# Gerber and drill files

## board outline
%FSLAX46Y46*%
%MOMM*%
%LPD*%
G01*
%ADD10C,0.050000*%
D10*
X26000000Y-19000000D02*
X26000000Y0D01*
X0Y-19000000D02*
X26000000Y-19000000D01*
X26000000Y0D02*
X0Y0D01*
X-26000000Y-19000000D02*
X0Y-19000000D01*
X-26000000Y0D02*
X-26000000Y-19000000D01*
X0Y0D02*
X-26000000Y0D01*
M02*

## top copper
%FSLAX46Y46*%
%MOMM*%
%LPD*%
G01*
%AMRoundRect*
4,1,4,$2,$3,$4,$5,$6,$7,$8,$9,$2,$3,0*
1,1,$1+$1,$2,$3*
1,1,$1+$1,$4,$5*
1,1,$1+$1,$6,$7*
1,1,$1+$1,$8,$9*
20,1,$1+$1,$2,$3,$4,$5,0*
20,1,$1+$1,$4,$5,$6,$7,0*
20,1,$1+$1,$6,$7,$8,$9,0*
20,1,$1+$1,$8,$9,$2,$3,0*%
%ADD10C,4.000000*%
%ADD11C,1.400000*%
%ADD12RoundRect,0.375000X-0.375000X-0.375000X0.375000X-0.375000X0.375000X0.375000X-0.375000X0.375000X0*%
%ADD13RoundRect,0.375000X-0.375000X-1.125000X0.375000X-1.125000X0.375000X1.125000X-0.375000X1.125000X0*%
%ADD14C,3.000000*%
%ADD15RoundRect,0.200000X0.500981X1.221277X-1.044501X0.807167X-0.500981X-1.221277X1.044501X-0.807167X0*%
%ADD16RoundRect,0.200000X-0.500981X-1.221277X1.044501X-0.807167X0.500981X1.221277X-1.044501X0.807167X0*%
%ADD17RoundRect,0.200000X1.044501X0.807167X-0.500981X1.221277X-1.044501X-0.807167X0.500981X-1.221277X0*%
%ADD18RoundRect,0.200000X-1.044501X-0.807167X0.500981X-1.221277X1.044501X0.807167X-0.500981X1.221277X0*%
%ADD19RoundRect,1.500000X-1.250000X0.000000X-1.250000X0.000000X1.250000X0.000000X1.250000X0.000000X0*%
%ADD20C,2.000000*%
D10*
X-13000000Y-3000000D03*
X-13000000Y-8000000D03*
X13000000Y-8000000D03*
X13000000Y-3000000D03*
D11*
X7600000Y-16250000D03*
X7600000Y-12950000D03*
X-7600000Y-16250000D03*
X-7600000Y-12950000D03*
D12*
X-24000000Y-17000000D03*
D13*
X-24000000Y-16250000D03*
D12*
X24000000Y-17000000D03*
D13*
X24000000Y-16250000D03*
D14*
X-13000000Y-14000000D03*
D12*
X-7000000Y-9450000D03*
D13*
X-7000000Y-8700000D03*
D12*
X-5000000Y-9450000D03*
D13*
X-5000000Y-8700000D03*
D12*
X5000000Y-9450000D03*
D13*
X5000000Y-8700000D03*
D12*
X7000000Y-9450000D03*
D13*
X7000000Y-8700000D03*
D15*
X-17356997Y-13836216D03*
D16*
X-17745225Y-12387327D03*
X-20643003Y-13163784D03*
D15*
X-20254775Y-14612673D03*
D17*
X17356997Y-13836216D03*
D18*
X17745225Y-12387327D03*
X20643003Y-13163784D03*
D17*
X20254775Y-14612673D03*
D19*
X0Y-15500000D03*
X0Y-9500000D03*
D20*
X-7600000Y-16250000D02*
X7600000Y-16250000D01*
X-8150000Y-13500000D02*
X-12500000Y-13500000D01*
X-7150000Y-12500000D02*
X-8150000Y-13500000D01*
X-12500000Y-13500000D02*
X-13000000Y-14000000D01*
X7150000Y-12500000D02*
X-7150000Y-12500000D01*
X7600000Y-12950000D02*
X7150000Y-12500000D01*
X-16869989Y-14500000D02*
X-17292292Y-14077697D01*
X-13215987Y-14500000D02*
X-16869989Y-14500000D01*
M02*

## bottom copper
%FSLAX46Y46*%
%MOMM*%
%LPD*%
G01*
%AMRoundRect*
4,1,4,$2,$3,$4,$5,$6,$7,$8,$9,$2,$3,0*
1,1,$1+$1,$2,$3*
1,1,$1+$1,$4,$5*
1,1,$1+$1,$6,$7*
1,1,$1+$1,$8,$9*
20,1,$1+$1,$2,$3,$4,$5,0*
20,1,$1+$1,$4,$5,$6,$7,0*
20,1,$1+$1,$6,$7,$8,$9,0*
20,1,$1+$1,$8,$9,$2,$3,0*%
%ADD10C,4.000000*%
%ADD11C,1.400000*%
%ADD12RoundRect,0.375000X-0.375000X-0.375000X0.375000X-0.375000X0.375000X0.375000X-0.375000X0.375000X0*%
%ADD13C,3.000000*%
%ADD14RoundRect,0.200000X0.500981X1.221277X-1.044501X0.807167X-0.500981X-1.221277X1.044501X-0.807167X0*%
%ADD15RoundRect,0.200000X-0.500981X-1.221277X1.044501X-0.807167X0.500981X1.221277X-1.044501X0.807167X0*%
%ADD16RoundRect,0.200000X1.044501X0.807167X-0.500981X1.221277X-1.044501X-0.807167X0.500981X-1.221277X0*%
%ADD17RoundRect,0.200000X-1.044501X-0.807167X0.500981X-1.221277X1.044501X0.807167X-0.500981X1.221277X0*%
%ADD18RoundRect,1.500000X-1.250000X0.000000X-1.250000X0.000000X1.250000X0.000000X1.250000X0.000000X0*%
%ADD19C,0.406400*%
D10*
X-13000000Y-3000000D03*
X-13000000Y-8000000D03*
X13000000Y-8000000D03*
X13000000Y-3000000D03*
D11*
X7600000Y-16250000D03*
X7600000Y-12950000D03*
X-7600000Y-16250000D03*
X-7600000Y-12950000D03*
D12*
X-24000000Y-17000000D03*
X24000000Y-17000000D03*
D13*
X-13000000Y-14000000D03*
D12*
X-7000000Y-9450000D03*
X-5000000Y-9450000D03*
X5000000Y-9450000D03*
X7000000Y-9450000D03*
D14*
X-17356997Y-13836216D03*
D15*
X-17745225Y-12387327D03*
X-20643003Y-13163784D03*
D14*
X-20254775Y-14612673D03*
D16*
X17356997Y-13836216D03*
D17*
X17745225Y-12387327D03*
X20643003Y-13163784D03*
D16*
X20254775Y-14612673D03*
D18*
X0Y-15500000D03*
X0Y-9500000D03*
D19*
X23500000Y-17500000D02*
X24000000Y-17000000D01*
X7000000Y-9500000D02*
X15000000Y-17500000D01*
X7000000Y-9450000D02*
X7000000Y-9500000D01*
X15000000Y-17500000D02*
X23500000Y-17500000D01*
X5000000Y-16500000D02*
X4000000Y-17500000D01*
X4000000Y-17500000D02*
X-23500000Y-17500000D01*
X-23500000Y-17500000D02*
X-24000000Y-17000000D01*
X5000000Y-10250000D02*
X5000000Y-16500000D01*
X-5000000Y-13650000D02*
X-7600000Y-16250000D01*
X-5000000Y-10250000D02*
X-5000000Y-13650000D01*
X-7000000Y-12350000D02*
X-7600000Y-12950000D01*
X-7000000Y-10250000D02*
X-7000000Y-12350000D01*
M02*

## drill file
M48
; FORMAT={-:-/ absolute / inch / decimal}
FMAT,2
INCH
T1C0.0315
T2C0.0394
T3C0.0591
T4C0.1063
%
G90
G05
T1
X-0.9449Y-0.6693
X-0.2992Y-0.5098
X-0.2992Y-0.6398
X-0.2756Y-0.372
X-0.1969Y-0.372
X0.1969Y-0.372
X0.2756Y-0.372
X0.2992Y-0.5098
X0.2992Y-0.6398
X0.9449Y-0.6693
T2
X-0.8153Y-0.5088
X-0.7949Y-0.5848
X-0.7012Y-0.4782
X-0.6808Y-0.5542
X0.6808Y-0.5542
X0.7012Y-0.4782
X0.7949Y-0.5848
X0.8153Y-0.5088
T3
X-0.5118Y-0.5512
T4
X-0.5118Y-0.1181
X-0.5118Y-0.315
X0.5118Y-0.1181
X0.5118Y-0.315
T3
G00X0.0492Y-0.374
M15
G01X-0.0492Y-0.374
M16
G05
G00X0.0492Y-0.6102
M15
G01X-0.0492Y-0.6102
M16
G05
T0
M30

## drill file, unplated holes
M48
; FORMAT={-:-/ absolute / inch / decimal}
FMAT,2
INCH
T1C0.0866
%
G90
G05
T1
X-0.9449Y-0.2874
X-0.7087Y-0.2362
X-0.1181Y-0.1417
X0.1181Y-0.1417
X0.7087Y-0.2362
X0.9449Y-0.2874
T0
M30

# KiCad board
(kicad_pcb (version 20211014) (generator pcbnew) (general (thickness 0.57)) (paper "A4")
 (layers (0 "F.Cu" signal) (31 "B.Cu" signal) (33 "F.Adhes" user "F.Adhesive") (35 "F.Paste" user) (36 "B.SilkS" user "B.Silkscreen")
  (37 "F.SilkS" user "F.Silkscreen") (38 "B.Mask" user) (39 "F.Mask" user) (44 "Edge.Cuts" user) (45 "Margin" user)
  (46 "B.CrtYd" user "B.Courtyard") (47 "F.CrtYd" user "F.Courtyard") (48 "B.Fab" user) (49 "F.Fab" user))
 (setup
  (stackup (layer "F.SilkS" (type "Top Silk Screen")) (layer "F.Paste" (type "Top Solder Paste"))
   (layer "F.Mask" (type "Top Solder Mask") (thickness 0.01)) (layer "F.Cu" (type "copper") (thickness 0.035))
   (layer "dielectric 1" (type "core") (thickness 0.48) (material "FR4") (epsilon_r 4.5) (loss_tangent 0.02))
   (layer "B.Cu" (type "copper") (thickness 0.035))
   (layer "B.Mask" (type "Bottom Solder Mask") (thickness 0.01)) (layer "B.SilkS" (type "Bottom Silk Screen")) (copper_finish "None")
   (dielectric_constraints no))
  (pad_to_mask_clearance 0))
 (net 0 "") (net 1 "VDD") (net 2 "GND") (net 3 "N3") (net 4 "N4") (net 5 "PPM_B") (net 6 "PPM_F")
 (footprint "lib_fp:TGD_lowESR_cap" (layer "F.Cu") (at -7.6 14.6 90)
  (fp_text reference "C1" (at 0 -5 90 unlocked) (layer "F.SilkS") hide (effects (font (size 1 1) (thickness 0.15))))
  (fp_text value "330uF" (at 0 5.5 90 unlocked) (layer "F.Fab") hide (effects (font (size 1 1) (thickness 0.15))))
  (pad "1" thru_hole circle (at -1.65 0 90) (size 1.4 1.4) (drill 0.8) (layers *.Cu *.Mask) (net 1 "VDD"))
  (pad "2" thru_hole circle (at 1.65 0 90) (size 1.4 1.4) (drill 0.8) (layers *.Cu *.Mask) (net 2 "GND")))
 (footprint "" (layer "F.Cu") (at -13 14)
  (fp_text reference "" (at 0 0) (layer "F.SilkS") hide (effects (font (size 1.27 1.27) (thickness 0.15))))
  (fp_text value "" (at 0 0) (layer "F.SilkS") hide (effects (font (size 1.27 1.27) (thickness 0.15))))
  (pad "2" thru_hole circle (at 0 0 270) (size 3 3) (drill 1.5) (layers *.Cu *.Mask) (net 2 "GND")))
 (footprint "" (layer "F.Cu") (at 24 7.3)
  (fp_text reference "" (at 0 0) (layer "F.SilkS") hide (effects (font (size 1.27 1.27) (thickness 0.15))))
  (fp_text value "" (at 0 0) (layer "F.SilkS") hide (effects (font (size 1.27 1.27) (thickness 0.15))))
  (pad "" np_thru_hole circle (at 0 0 270) (size 2.2 2.2) (drill 2.2) (layers F&B.Cu *.Mask)))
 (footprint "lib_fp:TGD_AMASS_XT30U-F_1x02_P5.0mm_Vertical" (layer "F.Cu") (at 13 5.5 90)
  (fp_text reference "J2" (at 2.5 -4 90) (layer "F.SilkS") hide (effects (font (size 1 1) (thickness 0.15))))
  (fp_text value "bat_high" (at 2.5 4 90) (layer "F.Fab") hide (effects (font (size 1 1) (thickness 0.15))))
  (pad "1" thru_hole circle (at -2.5 0 90) (size 4 4) (drill 2.7) (layers *.Cu *.Mask) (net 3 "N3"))
  (pad "2" thru_hole circle (at 2.5 0 90) (size 4 4) (drill 2.7) (layers *.Cu *.Mask) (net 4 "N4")))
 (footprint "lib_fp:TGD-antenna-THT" (layer "F.Cu") (at -5 8.7)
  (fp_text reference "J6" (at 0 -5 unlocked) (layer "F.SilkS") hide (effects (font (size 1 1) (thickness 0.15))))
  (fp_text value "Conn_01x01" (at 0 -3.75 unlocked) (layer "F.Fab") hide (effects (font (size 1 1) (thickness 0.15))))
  (pad "1" smd roundrect (at 0 0) (size 1.5 3) (layers "F.Cu" "F.Paste" "F.Mask") (roundrect_rratio 0.25) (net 1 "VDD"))
  (pad "1" thru_hole roundrect (at 0 0.75) (size 1.5 1.5) (drill 0.8) (layers *.Cu *.Mask) (roundrect_rratio 0.25) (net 1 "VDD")))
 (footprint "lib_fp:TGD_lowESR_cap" (layer "F.Cu") (at 7.6 14.6 90)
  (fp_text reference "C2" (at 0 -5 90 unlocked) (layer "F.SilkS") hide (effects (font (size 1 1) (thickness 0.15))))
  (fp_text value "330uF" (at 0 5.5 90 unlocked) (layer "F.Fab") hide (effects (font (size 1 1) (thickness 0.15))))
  (pad "1" thru_hole circle (at -1.65 0 90) (size 1.4 1.4) (drill 0.8) (layers *.Cu *.Mask) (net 1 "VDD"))
  (pad "2" thru_hole circle (at 1.65 0 90) (size 1.4 1.4) (drill 0.8) (layers *.Cu *.Mask) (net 2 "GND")))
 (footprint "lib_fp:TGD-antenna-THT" (layer "F.Cu") (at 5 8.7)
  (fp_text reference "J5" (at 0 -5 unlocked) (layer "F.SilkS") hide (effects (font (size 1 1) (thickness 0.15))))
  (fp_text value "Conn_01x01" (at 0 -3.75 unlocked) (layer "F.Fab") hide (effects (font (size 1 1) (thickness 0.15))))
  (pad "1" thru_hole roundrect (at 0 0.75) (size 1.5 1.5) (drill 0.8) (layers *.Cu *.Mask) (roundrect_rratio 0.25) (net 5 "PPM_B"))
  (pad "1" smd roundrect (at 0 0) (size 1.5 3) (layers "F.Cu" "F.Paste" "F.Mask") (roundrect_rratio 0.25) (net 5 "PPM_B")))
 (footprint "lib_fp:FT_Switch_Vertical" (layer "F.Cu") (at 0 9.5 -90)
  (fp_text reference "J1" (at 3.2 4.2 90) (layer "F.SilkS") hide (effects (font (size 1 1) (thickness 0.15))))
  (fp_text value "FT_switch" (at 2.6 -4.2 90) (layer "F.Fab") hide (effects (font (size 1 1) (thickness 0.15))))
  (pad "1" thru_hole roundrect locked (at 0 0 270) (size 3 5.5) (drill oval 1.5 4) (layers *.Cu *.Mask) (roundrect_rratio 0.5) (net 3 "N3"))
  (pad "2" thru_hole roundrect locked (at 6 0 270) (size 3 5.5) (drill oval 1.5 4) (layers *.Cu *.Mask) (roundrect_rratio 0.5) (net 1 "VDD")))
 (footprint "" (layer "F.Cu") (at -18 6)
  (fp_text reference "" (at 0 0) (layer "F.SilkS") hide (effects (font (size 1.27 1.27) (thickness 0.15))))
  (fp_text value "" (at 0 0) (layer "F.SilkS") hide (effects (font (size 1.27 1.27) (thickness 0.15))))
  (pad "" np_thru_hole circle (at 0 0 270) (size 2.2 2.2) (drill 2.2) (layers F&B.Cu *.Mask)))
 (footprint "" (layer "F.Cu") (at 3 3.6)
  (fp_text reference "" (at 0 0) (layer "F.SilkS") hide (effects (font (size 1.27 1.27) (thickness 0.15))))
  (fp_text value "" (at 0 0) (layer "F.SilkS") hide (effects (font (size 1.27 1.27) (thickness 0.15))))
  (pad "" np_thru_hole circle (at 0 0 270) (size 2.2 2.2) (drill 2.2) (layers F&B.Cu *.Mask)))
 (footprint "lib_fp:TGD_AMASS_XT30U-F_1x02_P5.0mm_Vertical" (layer "F.Cu") (at -13 5.5 -90)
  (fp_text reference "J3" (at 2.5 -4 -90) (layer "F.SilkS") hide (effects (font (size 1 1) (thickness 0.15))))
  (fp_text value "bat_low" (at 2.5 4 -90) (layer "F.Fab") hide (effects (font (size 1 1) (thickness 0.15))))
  (pad "1" thru_hole circle (at -2.5 0 270) (size 4 4) (drill 2.7) (layers *.Cu *.Mask) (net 4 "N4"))
  (pad "2" thru_hole circle (at 2.5 0 270) (size 4 4) (drill 2.7) (layers *.Cu *.Mask) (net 2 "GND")))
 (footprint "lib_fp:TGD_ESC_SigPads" (layer "F.Cu") (at 19 13.5 -15)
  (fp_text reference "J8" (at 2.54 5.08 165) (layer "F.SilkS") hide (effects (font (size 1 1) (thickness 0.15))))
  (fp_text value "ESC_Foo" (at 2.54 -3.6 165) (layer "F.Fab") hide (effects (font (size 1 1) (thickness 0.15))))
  (pad "1" thru_hole roundrect (at -1.5 1 165) (size 2 2.5) (drill 1 (offset 0 0.25)) (layers *.Cu *.Mask) (roundrect_rratio 0.1)
   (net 1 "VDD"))
  (pad "1" thru_hole roundrect (at -1.5 -1 345) (size 2 2.5) (drill 1 (offset 0 0.25)) (layers *.Cu *.Mask) (roundrect_rratio 0.1)
   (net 1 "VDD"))
  (pad "2" thru_hole roundrect (at 1.5 -1 345) (size 2 2.5) (drill 1 (offset 0 0.25)) (layers *.Cu *.Mask) (roundrect_rratio 0.1)
   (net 2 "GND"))
  (pad "2" thru_hole roundrect (at 1.5 1 165) (size 2 2.5) (drill 1 (offset 0 0.25)) (layers *.Cu *.Mask) (roundrect_rratio 0.1)
   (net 2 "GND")))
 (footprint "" (layer "F.Cu") (at 17.5 6)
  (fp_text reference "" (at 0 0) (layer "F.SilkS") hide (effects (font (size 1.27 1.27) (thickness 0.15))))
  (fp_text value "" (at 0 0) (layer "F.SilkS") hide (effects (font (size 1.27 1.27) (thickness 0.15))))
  (pad "" np_thru_hole circle (at 0.5 0 270) (size 2.2 2.2) (drill 2.2) (layers F&B.Cu *.Mask)))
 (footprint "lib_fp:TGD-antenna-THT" (layer "F.Cu") (at -7 8.7)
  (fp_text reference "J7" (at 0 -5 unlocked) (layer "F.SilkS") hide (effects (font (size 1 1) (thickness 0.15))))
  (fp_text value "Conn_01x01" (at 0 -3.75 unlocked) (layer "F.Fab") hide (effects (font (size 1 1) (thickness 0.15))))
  (pad "1" smd roundrect (at 0 0) (size 1.5 3) (layers "F.Cu" "F.Paste" "F.Mask") (roundrect_rratio 0.25) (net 2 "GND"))
  (pad "1" thru_hole roundrect (at 0 0.75) (size 1.5 1.5) (drill 0.8) (layers *.Cu *.Mask) (roundrect_rratio 0.25) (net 2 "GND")))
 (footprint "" (layer "F.Cu") (at -3 3.6)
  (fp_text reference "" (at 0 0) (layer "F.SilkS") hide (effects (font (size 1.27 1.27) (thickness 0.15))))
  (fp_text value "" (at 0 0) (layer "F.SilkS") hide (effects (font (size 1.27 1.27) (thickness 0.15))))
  (pad "" np_thru_hole circle (at 0 0 270) (size 2.2 2.2) (drill 2.2) (layers F&B.Cu *.Mask)))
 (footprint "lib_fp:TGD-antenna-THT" (layer "F.Cu") (at 7 8.7)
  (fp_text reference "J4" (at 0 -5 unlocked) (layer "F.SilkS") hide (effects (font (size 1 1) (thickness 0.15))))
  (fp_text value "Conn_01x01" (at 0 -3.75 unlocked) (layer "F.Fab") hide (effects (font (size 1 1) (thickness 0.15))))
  (pad "1" thru_hole roundrect (at 0 0.75) (size 1.5 1.5) (drill 0.8) (layers *.Cu *.Mask) (roundrect_rratio 0.25) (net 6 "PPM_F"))
  (pad "1" smd roundrect (at 0 0) (size 1.5 3) (layers "F.Cu" "F.Paste" "F.Mask") (roundrect_rratio 0.25) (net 6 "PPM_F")))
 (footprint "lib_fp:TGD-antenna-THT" (layer "F.Cu") (at -24 16.25)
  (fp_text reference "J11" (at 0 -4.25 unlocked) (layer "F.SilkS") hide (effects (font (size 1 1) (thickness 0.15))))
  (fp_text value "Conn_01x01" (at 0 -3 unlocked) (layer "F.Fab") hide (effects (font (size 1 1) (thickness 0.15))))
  (pad "1" thru_hole roundrect (at 0 0.75) (size 1.5 1.5) (drill 0.8) (layers *.Cu *.Mask) (roundrect_rratio 0.25) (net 5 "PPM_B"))
  (pad "1" smd roundrect (at 0 0) (size 1.5 3) (layers "F.Cu" "F.Paste" "F.Mask") (roundrect_rratio 0.25) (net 5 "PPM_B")))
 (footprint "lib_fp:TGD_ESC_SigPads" (layer "F.Cu") (at -19 13.5 15)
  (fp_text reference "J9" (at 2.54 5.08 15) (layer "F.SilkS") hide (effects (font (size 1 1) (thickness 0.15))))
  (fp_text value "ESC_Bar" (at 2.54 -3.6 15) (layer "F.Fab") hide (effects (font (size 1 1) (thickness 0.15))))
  (pad "1" thru_hole roundrect (at -1.5 1 195) (size 2 2.5) (drill 1 (offset 0 0.25)) (layers *.Cu *.Mask) (roundrect_rratio 0.1)
   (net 1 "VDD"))
  (pad "1" thru_hole roundrect (at -1.5 -1 15) (size 2 2.5) (drill 1 (offset 0 0.25)) (layers *.Cu *.Mask) (roundrect_rratio 0.1)
   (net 1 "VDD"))
  (pad "2" thru_hole roundrect (at 1.5 1 195) (size 2 2.5) (drill 1 (offset 0 0.25)) (layers *.Cu *.Mask) (roundrect_rratio 0.1)
   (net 2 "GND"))
  (pad "2" thru_hole roundrect (at 1.5 -1 15) (size 2 2.5) (drill 1 (offset 0 0.25)) (layers *.Cu *.Mask) (roundrect_rratio 0.1)
   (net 2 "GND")))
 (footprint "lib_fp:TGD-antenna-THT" (layer "F.Cu") (at 24 16.25)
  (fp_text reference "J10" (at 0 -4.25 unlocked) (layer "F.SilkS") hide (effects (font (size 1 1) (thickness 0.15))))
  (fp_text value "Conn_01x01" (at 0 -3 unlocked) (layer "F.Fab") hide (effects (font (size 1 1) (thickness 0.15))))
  (pad "1" smd roundrect (at 0 0) (size 1.5 3) (layers "F.Cu" "F.Paste" "F.Mask") (roundrect_rratio 0.25) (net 6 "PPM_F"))
  (pad "1" thru_hole roundrect (at 0 0.75) (size 1.5 1.5) (drill 0.8) (layers *.Cu *.Mask) (roundrect_rratio 0.25) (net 6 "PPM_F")))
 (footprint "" (layer "F.Cu") (at -24.5 7.3)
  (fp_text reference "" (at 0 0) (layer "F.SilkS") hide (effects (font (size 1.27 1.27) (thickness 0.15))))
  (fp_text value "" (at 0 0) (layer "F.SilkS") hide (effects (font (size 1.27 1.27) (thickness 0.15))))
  (pad "" np_thru_hole circle (at 0.5 0 270) (size 2.2 2.2) (drill 2.2) (layers F&B.Cu *.Mask)))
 (gr_line (start -26 0) (end -26 19) (layer "Edge.Cuts") (width 0.05))
 (gr_line (start 26 0) (end 0 0) (layer "Edge.Cuts") (width 0.05))
 (gr_line (start 0 0) (end -26 0) (layer "Edge.Cuts") (width 0.05))
 (gr_line (start 26 19) (end 26 0) (layer "Edge.Cuts") (width 0.05))
 (gr_line (start -26 19) (end 0 19) (layer "Edge.Cuts") (width 0.05))
 (gr_line (start 0 19) (end 26 19) (layer "Edge.Cuts") (width 0.05))
 (segment (start 7.6 12.95) (end 7.15 12.5) (width 2) (layer "F.Cu") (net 2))
 (segment (start -8.15 13.5) (end -12.5 13.5) (width 2) (layer "F.Cu") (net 2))
 (segment (start -13.215987 14.5) (end -16.869989 14.5) (width 2) (layer "F.Cu") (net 2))
 (segment (start -16.869989 14.5) (end -17.292292 14.077697) (width 2) (layer "F.Cu") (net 2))
 (segment (start -12.5 13.5) (end -13 14) (width 2) (layer "F.Cu") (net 2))
 (segment (start -7.15 12.5) (end -8.15 13.5) (width 2) (layer "F.Cu") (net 2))
 (segment (start 7.15 12.5) (end -7.15 12.5) (width 2) (layer "F.Cu") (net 2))
 (segment (start -7 12.35) (end -7.6 12.95) (width 0.4064) (layer "B.Cu") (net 2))
 (segment (start -7 10.25) (end -7 12.35) (width 0.4064) (layer "B.Cu") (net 2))
 (segment (start -7.6 16.25) (end 7.6 16.25) (width 2) (layer "F.Cu") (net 1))
 (segment (start -5 10.25) (end -5 13.65) (width 0.4064) (layer "B.Cu") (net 1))
 (segment (start -5 13.65) (end -7.6 16.25) (width 0.4064) (layer "B.Cu") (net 1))
 (segment (start 23.5 17.5) (end 24 17) (width 0.4064) (layer "B.Cu") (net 6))
 (segment (start 15 17.5) (end 23.5 17.5) (width 0.4064) (layer "B.Cu") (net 6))
 (segment (start 7 9.5) (end 15 17.5) (width 0.4064) (layer "B.Cu") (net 6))
 (segment (start 7 9.45) (end 7 9.5) (width 0.4064) (layer "B.Cu") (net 6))
 (segment (start -23.5 17.5) (end -24 17) (width 0.4064) (layer "B.Cu") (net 5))
 (segment (start 5 16.5) (end 4 17.5) (width 0.4064) (layer "B.Cu") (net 5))
 (segment (start 5 10.25) (end 5 16.5) (width 0.4064) (layer "B.Cu") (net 5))
 (segment (start 4 17.5) (end -23.5 17.5) (width 0.4064) (layer "B.Cu") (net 5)))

